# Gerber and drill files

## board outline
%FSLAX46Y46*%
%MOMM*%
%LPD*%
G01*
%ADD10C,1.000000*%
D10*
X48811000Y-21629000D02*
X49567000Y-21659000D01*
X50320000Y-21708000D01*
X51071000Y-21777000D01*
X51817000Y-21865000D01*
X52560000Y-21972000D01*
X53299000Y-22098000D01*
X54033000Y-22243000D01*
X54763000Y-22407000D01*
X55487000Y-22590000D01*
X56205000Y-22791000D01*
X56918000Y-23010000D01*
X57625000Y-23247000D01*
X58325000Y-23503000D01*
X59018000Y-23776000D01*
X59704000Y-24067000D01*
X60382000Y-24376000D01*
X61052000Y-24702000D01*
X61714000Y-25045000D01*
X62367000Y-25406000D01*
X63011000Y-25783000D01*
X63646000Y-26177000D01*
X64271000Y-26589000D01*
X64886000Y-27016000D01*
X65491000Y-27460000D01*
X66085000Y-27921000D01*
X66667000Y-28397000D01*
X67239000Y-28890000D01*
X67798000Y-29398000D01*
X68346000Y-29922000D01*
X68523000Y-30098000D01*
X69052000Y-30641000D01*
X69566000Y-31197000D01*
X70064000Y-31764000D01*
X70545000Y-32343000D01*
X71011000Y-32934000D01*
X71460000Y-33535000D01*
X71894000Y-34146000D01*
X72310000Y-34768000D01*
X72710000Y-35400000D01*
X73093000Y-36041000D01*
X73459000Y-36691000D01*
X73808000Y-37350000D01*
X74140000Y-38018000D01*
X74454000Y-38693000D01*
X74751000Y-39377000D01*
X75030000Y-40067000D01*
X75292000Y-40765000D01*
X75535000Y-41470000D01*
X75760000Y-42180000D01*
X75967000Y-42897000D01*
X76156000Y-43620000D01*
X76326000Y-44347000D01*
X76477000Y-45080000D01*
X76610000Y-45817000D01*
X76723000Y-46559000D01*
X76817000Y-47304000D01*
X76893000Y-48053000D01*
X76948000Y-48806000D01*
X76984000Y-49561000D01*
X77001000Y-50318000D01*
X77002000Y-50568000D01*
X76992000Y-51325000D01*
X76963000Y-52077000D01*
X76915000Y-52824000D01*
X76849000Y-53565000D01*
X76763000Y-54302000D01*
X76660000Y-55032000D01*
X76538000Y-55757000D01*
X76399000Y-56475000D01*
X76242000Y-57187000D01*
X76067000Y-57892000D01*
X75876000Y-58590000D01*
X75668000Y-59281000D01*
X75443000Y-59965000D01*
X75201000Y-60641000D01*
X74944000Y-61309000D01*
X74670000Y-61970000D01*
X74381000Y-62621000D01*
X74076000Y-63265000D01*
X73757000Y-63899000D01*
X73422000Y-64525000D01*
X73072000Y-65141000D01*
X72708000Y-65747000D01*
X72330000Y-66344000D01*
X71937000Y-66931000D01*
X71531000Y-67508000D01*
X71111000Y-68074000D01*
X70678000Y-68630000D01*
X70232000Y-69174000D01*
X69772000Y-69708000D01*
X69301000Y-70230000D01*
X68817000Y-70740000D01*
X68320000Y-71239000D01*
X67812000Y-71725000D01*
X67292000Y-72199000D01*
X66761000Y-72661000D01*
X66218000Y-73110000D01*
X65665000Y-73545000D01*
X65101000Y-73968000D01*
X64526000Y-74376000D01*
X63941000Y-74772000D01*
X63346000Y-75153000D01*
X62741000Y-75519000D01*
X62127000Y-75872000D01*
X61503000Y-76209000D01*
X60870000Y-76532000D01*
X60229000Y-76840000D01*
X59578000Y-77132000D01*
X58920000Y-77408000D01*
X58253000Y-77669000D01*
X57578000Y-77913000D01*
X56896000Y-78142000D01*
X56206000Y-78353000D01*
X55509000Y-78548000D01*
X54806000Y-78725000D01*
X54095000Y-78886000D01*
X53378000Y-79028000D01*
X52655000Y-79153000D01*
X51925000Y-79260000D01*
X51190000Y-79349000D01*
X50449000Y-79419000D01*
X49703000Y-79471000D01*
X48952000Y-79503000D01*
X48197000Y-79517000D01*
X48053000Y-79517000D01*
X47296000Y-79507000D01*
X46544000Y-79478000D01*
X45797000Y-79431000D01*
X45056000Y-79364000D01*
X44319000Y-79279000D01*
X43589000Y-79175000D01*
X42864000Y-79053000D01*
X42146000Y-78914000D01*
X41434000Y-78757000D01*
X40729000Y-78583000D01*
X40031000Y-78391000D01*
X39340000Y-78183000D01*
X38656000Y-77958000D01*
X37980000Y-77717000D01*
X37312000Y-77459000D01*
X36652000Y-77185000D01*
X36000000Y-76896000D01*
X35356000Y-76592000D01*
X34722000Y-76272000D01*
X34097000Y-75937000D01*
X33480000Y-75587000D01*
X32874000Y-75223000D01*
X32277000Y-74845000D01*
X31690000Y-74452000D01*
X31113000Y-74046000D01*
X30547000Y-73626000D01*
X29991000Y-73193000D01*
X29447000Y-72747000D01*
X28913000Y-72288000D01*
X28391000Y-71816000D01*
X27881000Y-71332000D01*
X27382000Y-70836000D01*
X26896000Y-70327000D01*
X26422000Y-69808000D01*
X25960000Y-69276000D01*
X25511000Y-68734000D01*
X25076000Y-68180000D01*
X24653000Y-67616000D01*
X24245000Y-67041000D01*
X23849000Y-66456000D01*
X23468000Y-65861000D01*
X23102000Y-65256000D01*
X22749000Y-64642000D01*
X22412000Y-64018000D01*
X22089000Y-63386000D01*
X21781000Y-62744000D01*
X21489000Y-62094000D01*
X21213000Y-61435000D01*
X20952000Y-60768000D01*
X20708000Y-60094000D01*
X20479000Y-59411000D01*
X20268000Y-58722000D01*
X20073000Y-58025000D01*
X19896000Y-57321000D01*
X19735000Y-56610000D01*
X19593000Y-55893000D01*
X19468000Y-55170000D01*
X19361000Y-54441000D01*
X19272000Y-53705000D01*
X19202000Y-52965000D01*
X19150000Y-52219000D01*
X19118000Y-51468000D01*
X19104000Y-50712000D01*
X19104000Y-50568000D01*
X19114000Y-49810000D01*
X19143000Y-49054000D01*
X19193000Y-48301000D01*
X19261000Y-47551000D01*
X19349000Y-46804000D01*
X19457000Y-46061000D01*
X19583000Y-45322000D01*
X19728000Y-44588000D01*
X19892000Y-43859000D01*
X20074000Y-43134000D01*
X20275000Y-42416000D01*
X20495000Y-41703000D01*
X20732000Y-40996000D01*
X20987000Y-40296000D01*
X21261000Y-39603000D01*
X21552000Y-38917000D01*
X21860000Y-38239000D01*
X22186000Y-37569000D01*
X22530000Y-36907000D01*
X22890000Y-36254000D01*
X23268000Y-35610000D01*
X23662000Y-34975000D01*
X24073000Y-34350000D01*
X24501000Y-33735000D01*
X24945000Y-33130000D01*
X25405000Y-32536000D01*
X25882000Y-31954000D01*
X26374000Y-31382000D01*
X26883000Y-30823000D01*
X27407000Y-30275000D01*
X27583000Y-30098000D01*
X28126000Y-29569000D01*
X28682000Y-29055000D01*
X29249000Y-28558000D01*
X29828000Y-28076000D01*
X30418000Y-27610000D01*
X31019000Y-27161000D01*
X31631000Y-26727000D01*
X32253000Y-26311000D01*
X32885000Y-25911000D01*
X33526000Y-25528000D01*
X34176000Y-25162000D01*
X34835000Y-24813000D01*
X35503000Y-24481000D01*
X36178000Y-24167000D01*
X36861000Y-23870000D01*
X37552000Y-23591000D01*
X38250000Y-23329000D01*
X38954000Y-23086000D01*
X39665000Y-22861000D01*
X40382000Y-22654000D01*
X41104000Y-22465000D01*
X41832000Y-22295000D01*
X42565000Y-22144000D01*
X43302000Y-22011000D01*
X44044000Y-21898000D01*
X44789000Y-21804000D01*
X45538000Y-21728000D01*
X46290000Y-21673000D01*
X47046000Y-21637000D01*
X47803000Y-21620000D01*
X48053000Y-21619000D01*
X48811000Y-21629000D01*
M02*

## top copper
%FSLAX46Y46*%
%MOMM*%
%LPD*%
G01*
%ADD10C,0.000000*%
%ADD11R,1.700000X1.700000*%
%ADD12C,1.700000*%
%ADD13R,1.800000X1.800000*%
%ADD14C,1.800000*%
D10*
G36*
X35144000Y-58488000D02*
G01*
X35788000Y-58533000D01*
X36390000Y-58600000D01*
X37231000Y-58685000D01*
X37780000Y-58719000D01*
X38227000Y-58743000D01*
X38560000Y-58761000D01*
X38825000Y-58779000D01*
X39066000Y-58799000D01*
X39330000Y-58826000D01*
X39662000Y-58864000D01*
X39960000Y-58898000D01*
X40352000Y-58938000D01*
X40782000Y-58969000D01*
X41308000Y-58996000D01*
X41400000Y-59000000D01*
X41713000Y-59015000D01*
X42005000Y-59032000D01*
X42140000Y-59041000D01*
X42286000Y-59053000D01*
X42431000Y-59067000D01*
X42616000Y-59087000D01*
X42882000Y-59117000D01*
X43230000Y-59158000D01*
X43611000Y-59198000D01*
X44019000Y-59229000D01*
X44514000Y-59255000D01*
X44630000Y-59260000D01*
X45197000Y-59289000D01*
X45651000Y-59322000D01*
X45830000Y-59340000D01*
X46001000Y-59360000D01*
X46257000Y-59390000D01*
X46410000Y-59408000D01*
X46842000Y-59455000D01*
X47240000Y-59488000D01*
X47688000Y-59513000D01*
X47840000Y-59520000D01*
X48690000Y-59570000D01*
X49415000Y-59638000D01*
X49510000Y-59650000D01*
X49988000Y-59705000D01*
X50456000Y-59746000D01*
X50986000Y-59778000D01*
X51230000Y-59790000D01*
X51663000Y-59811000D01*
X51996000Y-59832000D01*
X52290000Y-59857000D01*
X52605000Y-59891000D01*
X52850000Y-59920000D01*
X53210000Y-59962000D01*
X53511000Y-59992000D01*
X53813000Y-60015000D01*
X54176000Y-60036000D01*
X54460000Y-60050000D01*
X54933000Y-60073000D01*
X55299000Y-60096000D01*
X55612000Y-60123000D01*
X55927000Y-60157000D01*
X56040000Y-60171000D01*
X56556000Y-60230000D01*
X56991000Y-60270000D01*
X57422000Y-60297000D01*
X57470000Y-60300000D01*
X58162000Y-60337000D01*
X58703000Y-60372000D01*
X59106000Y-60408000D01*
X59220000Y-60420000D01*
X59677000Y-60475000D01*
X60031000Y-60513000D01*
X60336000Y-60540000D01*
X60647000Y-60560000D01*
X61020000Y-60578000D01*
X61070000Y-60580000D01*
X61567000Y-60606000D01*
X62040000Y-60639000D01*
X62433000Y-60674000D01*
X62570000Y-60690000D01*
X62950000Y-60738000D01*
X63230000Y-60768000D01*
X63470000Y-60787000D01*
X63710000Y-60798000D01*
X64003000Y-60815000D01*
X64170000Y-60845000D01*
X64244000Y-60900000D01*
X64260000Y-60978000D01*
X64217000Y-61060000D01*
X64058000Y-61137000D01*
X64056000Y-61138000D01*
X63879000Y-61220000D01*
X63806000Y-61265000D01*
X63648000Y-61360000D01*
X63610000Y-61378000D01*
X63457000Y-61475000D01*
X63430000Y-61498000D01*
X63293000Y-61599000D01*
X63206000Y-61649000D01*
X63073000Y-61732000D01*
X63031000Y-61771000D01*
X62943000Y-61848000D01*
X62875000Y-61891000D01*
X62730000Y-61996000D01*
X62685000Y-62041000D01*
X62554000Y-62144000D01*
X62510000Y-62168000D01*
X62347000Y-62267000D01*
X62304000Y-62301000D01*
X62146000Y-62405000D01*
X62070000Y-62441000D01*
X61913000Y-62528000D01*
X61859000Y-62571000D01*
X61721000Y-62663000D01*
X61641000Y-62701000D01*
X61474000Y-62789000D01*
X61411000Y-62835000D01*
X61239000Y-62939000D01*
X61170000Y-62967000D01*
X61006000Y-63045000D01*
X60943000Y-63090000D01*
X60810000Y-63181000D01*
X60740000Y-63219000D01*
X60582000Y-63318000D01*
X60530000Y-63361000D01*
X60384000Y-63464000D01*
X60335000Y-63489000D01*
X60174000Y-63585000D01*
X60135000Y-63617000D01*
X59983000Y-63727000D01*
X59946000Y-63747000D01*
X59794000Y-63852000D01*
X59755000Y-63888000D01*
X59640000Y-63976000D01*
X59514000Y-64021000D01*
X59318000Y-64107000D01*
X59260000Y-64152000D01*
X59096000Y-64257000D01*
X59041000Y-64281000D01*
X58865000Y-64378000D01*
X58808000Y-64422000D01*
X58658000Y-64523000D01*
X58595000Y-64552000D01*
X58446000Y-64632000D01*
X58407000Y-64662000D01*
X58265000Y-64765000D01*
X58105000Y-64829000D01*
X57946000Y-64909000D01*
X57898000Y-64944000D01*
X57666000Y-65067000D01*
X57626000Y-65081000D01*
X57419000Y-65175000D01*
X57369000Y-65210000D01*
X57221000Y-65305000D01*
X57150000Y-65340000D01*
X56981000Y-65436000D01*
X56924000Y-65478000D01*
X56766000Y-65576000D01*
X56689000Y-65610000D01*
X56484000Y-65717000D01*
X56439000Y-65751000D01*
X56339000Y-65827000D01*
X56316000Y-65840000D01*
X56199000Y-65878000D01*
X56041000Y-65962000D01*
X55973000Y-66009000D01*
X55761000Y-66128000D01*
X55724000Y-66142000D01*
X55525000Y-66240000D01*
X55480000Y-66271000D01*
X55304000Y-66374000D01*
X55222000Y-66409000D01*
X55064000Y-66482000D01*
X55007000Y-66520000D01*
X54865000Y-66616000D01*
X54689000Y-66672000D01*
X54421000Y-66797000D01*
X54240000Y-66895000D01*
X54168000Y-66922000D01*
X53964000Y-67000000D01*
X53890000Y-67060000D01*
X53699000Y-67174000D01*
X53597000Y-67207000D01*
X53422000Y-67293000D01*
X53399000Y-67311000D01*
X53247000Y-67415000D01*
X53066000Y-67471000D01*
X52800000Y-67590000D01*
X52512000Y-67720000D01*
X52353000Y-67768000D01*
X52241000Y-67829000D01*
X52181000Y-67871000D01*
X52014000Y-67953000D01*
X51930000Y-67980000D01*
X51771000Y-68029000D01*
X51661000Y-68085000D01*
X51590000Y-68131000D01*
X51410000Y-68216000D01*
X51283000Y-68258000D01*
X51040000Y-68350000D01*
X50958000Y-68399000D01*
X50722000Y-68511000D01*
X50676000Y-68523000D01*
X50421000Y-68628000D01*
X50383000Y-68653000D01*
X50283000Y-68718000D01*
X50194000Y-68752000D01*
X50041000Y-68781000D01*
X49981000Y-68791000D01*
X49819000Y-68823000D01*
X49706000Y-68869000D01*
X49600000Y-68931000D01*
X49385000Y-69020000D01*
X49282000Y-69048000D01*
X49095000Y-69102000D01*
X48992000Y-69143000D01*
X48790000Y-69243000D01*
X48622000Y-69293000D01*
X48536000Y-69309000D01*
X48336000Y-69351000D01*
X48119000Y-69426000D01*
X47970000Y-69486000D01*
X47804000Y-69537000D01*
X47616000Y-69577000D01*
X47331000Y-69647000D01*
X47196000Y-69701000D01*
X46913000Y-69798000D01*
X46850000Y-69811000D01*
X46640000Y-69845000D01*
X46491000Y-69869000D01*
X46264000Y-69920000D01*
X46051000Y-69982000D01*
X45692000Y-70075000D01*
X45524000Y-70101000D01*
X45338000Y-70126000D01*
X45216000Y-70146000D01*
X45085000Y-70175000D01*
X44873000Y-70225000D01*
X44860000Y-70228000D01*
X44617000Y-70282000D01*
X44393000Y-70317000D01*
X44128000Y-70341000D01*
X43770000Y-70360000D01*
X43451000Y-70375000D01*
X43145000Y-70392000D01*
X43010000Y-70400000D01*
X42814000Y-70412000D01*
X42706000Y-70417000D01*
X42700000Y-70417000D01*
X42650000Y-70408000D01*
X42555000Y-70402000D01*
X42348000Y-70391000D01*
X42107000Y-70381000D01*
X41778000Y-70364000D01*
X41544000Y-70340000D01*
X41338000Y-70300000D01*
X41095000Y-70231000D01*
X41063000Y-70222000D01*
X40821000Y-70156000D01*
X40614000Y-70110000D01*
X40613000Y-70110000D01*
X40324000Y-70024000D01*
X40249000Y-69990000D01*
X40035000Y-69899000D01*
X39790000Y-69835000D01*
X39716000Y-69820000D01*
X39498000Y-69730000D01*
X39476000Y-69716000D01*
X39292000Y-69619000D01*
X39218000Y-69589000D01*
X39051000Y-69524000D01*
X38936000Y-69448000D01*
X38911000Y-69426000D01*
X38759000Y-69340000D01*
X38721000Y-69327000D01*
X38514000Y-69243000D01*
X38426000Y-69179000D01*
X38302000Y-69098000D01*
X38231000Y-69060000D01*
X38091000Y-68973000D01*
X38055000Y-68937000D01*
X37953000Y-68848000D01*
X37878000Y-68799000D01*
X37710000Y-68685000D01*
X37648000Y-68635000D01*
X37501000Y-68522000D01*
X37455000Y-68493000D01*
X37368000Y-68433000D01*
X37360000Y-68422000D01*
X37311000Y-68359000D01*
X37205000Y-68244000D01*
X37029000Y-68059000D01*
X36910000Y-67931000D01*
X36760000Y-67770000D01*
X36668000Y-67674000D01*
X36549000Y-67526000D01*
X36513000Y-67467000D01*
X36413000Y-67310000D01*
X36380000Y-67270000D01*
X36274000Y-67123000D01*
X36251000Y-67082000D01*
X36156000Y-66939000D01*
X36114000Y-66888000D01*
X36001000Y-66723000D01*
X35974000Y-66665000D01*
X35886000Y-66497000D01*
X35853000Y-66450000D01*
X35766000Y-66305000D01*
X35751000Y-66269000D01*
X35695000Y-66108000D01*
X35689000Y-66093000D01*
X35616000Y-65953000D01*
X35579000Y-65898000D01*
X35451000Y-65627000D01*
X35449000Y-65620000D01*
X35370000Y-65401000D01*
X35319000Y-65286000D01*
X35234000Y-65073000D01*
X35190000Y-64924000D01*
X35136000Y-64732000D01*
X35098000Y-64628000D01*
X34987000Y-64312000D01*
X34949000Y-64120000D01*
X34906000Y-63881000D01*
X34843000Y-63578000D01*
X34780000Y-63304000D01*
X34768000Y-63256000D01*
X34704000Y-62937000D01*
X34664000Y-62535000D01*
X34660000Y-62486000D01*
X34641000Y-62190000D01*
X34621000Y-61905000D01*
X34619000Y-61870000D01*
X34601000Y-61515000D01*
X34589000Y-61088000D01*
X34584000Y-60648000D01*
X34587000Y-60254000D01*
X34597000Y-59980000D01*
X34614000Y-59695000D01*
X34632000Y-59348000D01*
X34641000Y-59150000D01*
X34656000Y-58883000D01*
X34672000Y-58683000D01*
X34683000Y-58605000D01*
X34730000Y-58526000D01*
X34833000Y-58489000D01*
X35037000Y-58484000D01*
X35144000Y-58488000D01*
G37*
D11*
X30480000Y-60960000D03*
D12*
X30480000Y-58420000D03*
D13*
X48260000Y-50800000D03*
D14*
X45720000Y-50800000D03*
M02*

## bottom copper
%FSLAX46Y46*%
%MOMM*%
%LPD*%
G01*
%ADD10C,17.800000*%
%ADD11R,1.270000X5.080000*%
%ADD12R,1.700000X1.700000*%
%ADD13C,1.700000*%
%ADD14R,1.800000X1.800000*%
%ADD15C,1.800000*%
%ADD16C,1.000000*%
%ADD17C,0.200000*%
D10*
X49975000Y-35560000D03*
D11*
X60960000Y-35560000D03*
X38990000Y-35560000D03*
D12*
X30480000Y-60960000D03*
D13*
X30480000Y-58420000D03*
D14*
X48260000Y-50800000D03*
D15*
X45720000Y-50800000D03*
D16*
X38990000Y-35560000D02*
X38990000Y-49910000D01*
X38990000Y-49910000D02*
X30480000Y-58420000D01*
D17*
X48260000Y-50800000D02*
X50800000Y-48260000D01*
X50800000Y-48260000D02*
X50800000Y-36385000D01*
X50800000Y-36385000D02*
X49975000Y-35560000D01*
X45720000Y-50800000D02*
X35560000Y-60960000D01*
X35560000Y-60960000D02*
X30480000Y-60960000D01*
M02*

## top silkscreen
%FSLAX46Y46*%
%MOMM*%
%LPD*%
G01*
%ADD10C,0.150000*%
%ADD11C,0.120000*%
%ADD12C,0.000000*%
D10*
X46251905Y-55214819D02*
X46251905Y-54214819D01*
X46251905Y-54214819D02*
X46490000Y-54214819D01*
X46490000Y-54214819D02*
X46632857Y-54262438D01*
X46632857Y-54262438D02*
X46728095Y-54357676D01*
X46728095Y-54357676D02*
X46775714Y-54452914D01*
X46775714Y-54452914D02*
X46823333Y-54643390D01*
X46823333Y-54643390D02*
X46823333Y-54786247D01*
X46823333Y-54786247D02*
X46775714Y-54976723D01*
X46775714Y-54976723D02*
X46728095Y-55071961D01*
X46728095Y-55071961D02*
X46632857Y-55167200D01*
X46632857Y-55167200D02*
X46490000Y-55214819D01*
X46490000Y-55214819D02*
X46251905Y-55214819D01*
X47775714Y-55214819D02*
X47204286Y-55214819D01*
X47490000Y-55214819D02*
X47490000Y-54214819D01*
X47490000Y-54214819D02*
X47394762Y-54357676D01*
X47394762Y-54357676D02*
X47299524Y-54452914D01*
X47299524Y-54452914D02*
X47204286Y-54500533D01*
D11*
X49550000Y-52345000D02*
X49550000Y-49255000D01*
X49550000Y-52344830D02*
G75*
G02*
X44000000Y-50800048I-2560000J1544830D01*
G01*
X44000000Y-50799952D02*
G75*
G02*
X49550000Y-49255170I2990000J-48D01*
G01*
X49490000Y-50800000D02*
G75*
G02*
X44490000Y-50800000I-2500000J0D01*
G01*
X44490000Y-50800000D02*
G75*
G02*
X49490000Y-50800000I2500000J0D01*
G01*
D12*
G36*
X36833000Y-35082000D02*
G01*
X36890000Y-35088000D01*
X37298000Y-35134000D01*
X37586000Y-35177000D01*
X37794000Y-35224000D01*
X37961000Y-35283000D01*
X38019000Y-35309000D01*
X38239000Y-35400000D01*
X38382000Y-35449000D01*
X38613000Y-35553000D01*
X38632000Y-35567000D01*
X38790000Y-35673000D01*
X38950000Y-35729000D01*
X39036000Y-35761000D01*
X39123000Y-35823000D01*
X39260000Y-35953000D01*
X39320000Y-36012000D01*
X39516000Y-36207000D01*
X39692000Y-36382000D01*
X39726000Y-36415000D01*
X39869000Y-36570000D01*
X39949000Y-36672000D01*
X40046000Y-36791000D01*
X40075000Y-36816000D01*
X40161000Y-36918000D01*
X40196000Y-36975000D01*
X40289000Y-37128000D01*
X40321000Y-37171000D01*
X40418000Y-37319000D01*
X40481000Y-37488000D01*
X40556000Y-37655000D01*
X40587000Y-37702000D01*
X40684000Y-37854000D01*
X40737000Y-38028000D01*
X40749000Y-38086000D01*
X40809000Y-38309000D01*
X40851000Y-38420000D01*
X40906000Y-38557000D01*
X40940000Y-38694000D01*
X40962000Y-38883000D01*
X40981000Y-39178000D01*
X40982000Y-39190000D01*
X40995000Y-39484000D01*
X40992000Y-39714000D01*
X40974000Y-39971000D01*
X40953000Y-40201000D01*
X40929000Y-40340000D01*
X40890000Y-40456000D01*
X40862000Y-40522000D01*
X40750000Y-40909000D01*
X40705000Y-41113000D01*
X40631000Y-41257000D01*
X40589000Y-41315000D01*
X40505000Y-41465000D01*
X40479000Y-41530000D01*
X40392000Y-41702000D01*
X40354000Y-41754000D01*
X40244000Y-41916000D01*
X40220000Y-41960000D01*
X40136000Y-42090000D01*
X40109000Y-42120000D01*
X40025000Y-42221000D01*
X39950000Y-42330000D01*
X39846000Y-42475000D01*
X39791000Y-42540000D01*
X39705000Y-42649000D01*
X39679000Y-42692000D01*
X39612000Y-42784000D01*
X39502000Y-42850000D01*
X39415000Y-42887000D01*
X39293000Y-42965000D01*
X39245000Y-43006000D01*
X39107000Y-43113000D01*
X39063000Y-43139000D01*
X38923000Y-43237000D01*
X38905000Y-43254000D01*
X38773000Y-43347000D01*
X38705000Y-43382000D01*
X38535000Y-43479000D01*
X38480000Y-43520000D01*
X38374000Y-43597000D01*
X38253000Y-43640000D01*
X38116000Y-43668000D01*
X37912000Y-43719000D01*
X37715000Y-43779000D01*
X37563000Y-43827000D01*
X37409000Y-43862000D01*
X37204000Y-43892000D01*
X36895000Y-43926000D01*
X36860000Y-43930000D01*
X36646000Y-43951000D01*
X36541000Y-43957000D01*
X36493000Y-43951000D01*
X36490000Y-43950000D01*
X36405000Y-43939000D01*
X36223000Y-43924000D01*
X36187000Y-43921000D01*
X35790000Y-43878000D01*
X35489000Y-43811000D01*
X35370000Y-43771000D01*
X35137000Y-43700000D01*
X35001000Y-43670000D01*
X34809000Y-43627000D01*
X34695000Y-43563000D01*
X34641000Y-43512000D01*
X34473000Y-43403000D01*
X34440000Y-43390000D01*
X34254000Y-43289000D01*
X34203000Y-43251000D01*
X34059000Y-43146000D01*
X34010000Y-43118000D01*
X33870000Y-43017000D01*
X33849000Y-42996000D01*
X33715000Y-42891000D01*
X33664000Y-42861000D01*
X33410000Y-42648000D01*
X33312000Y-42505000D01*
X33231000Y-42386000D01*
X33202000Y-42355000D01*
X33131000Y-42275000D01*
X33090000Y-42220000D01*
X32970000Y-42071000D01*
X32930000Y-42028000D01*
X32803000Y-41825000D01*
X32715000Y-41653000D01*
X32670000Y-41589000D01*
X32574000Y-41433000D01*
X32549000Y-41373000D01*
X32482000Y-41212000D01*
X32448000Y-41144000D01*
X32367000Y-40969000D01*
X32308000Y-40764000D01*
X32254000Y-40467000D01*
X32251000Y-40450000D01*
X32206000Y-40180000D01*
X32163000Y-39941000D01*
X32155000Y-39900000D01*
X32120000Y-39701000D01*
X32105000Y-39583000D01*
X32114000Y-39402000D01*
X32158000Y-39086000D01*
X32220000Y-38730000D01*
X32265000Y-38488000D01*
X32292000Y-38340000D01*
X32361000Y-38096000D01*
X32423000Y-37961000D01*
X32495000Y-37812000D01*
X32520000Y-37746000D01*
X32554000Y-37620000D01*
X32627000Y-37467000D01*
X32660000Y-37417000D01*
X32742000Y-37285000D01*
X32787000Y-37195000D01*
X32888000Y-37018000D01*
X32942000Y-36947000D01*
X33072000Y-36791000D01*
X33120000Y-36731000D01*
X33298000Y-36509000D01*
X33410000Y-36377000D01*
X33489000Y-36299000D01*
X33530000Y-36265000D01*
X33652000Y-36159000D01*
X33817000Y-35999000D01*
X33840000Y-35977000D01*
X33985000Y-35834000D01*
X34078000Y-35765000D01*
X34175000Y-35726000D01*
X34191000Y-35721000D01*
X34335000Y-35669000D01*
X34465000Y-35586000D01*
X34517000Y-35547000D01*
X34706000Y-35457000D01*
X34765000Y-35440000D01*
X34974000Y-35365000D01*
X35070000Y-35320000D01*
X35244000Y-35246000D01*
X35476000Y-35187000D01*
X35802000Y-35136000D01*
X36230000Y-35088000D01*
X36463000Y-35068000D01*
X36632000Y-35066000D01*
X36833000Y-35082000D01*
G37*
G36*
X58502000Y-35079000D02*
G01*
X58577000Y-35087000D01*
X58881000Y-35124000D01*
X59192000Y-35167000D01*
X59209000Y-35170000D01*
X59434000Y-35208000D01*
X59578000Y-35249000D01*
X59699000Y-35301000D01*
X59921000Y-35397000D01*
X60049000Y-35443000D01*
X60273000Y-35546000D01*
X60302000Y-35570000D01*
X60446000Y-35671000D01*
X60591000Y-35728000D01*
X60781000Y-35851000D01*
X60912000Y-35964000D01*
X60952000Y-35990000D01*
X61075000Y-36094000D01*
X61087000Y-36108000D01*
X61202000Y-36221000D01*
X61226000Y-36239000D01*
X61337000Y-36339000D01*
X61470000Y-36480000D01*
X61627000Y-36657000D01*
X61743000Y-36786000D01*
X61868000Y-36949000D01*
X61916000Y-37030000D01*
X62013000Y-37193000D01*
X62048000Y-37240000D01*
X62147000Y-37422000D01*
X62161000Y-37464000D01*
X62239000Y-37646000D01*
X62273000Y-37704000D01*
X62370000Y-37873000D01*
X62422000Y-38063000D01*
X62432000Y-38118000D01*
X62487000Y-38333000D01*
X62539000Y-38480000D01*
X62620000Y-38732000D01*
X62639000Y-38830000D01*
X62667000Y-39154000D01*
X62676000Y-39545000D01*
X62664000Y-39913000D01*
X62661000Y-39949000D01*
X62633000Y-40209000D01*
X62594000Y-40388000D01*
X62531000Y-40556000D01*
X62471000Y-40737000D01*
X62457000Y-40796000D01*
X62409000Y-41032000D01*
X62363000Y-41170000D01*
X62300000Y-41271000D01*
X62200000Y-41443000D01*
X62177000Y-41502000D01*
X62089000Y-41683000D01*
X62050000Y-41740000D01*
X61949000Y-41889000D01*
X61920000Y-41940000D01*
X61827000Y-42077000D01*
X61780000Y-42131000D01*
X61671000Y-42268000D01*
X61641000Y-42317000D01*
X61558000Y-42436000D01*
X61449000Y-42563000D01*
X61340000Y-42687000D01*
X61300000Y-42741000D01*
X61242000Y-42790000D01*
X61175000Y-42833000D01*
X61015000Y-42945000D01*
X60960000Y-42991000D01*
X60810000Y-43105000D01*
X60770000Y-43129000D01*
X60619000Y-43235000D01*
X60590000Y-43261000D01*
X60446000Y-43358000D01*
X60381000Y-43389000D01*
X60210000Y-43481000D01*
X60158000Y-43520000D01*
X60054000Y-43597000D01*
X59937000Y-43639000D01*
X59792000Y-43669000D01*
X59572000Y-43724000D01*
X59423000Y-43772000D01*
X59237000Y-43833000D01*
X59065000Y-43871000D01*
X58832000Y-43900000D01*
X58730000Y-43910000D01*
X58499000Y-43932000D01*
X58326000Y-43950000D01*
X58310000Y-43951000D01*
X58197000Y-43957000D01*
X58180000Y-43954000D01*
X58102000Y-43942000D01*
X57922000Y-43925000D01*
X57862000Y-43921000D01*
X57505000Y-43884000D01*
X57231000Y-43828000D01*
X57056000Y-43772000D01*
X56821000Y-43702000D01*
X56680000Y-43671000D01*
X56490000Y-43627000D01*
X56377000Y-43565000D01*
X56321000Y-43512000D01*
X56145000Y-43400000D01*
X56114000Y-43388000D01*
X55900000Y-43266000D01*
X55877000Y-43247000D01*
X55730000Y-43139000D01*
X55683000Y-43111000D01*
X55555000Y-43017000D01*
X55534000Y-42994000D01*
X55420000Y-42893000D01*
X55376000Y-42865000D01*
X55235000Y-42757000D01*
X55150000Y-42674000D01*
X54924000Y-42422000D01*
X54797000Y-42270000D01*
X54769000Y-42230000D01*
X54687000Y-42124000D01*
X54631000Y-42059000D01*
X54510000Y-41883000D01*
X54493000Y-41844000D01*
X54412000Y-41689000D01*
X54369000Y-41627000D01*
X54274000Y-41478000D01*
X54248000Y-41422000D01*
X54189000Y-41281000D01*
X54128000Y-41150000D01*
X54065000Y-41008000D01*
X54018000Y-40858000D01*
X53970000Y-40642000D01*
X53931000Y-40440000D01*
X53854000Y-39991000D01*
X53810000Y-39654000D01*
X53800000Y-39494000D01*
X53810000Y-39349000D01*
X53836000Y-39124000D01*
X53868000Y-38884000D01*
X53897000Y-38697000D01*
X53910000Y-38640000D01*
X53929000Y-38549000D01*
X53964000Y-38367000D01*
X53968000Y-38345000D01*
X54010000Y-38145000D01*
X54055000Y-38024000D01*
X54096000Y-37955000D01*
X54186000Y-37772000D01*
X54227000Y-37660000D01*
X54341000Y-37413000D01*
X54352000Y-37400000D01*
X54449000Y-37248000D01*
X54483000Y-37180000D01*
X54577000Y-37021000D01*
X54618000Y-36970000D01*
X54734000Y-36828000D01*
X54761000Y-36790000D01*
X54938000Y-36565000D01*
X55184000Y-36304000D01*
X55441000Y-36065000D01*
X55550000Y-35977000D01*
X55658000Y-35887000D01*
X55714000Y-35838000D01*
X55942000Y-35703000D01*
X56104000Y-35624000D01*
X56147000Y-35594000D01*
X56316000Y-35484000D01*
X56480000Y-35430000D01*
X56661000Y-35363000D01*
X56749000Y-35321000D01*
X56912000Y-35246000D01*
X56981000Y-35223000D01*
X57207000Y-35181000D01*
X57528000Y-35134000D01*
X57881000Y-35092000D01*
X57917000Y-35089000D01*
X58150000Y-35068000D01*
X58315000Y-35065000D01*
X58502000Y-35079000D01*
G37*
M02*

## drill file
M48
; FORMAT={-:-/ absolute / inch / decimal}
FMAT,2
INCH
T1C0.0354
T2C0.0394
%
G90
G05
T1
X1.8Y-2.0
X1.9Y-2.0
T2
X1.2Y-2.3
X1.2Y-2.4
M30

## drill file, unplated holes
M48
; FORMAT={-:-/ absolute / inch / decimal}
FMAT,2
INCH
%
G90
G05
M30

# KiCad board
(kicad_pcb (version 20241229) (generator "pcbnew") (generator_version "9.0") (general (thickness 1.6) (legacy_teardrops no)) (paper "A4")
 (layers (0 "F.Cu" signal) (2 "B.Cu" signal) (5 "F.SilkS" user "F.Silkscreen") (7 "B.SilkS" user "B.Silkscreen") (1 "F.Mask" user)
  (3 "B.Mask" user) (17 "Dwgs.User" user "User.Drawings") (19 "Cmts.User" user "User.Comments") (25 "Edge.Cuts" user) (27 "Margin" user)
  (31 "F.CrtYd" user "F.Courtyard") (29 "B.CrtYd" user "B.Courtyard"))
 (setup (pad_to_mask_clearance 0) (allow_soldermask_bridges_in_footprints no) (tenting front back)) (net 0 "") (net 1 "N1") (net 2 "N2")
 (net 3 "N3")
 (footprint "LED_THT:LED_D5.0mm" (layer "F.Cu") (at 48.26 50.8 180)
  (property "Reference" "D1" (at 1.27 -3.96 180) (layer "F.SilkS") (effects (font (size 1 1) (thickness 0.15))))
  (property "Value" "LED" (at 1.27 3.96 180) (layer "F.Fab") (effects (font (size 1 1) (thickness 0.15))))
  (fp_line (start -1.29 -1.545) (end -1.29 1.545) (stroke (width 0.12) (type solid)) (layer "F.SilkS"))
  (fp_arc (start 4.26 0.000048) (mid 2.071756 2.880501) (end -1.29 1.54483) (stroke (width 0.12) (type solid)) (layer "F.SilkS"))
  (fp_arc (start -1.29 -1.54483) (mid 2.071756 -2.880501) (end 4.26 -0.000048) (stroke (width 0.12) (type solid)) (layer "F.SilkS"))
  (fp_circle (center 1.27 0) (end 3.77 0) (stroke (width 0.12) (type solid)) (fill no) (layer "F.SilkS"))
  (pad "1" thru_hole rect (at 0 0 180) (size 1.8 1.8) (drill 0.9) (layers "*.Cu" "*.Mask") (remove_unused_layers no) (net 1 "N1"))
  (pad "2" thru_hole circle (at 2.54 0 180) (size 1.8 1.8) (drill 0.9) (layers "*.Cu" "*.Mask") (remove_unused_layers no) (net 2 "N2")))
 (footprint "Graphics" (layer "F.Cu") (at 0 0)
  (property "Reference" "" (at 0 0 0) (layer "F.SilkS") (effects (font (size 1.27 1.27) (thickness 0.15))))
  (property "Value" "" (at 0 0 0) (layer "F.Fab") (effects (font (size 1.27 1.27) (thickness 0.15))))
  (fp_poly
   (pts (xy 35.144 58.488) (xy 35.788 58.533) (xy 36.39 58.6) (xy 37.231 58.685) (xy 37.78 58.719) (xy 38.227 58.743) (xy 38.56 58.761)
    (xy 38.825 58.779) (xy 39.066 58.799) (xy 39.33 58.826) (xy 39.662 58.864) (xy 39.96 58.898) (xy 40.352 58.938) (xy 40.782 58.969)
    (xy 41.308 58.996) (xy 41.4 59) (xy 41.713 59.015) (xy 42.005 59.032) (xy 42.14 59.041) (xy 42.286 59.053) (xy 42.431 59.067)
    (xy 42.616 59.087) (xy 42.882 59.117) (xy 43.23 59.158) (xy 43.611 59.198) (xy 44.019 59.229) (xy 44.514 59.255) (xy 44.63 59.26)
    (xy 45.197 59.289) (xy 45.651 59.322) (xy 45.83 59.34) (xy 46.001 59.36) (xy 46.257 59.39) (xy 46.41 59.408) (xy 46.842 59.455)
    (xy 47.24 59.488) (xy 47.688 59.513) (xy 47.84 59.52) (xy 48.69 59.57) (xy 49.415 59.638) (xy 49.51 59.65) (xy 49.988 59.705)
    (xy 50.456 59.746) (xy 50.986 59.778) (xy 51.23 59.79) (xy 51.663 59.811) (xy 51.996 59.832) (xy 52.29 59.857) (xy 52.605 59.891)
    (xy 52.85 59.92) (xy 53.21 59.962) (xy 53.511 59.992) (xy 53.813 60.015) (xy 54.176 60.036) (xy 54.46 60.05) (xy 54.933 60.073)
    (xy 55.299 60.096) (xy 55.612 60.123) (xy 55.927 60.157) (xy 56.04 60.171) (xy 56.556 60.23) (xy 56.991 60.27) (xy 57.422 60.297)
    (xy 57.47 60.3) (xy 58.162 60.337) (xy 58.703 60.372) (xy 59.106 60.408) (xy 59.22 60.42) (xy 59.677 60.475) (xy 60.031 60.513)
    (xy 60.336 60.54) (xy 60.647 60.56) (xy 61.02 60.578) (xy 61.07 60.58) (xy 61.567 60.606) (xy 62.04 60.639) (xy 62.433 60.674)
    (xy 62.57 60.69) (xy 62.95 60.738) (xy 63.23 60.768) (xy 63.47 60.787) (xy 63.71 60.798) (xy 64.003 60.815) (xy 64.17 60.845)
    (xy 64.244 60.9) (xy 64.26 60.978) (xy 64.217 61.06) (xy 64.058 61.137) (xy 64.056 61.138) (xy 63.879 61.22) (xy 63.806 61.265)
    (xy 63.648 61.36) (xy 63.61 61.378) (xy 63.457 61.475) (xy 63.43 61.498) (xy 63.293 61.599) (xy 63.206 61.649) (xy 63.073 61.732)
    (xy 63.031 61.771) (xy 62.943 61.848) (xy 62.875 61.891) (xy 62.73 61.996) (xy 62.685 62.041) (xy 62.554 62.144) (xy 62.51 62.168)
    (xy 62.347 62.267) (xy 62.304 62.301) (xy 62.146 62.405) (xy 62.07 62.441) (xy 61.913 62.528) (xy 61.859 62.571) (xy 61.721 62.663)
    (xy 61.641 62.701) (xy 61.474 62.789) (xy 61.411 62.835) (xy 61.239 62.939) (xy 61.17 62.967) (xy 61.006 63.045) (xy 60.943 63.09)
    (xy 60.81 63.181) (xy 60.74 63.219) (xy 60.582 63.318) (xy 60.53 63.361) (xy 60.384 63.464) (xy 60.335 63.489) (xy 60.174 63.585)
    (xy 60.135 63.617) (xy 59.983 63.727) (xy 59.946 63.747) (xy 59.794 63.852) (xy 59.755 63.888) (xy 59.64 63.976) (xy 59.514 64.021)
    (xy 59.318 64.107) (xy 59.26 64.152) (xy 59.096 64.257) (xy 59.041 64.281) (xy 58.865 64.378) (xy 58.808 64.422) (xy 58.658 64.523)
    (xy 58.595 64.552) (xy 58.446 64.632) (xy 58.407 64.662) (xy 58.265 64.765) (xy 58.105 64.829) (xy 57.946 64.909) (xy 57.898 64.944)
    (xy 57.666 65.067) (xy 57.626 65.081) (xy 57.419 65.175) (xy 57.369 65.21) (xy 57.221 65.305) (xy 57.15 65.34) (xy 56.981 65.436)
    (xy 56.924 65.478) (xy 56.766 65.576) (xy 56.689 65.61) (xy 56.484 65.717) (xy 56.439 65.751) (xy 56.339 65.827) (xy 56.316 65.84)
    (xy 56.199 65.878) (xy 56.041 65.962) (xy 55.973 66.009) (xy 55.761 66.128) (xy 55.724 66.142) (xy 55.525 66.24) (xy 55.48 66.271)
    (xy 55.304 66.374) (xy 55.222 66.409) (xy 55.064 66.482) (xy 55.007 66.52) (xy 54.865 66.616) (xy 54.689 66.672) (xy 54.421 66.797)
    (xy 54.24 66.895) (xy 54.168 66.922) (xy 53.964 67) (xy 53.89 67.06) (xy 53.699 67.174) (xy 53.597 67.207) (xy 53.422 67.293)
    (xy 53.399 67.311) (xy 53.247 67.415) (xy 53.066 67.471) (xy 52.8 67.59) (xy 52.512 67.72) (xy 52.353 67.768) (xy 52.241 67.829)
    (xy 52.181 67.871) (xy 52.014 67.953) (xy 51.93 67.98) (xy 51.771 68.029) (xy 51.661 68.085) (xy 51.59 68.131) (xy 51.41 68.216)
    (xy 51.283 68.258) (xy 51.04 68.35) (xy 50.958 68.399) (xy 50.722 68.511) (xy 50.676 68.523) (xy 50.421 68.628) (xy 50.383 68.653)
    (xy 50.283 68.718) (xy 50.194 68.752) (xy 50.041 68.781) (xy 49.981 68.791) (xy 49.819 68.823) (xy 49.706 68.869) (xy 49.6 68.931)
    (xy 49.385 69.02) (xy 49.282 69.048) (xy 49.095 69.102) (xy 48.992 69.143) (xy 48.79 69.243) (xy 48.622 69.293) (xy 48.536 69.309)
    (xy 48.336 69.351) (xy 48.119 69.426) (xy 47.97 69.486) (xy 47.804 69.537) (xy 47.616 69.577) (xy 47.331 69.647) (xy 47.196 69.701)
    (xy 46.913 69.798) (xy 46.85 69.811) (xy 46.64 69.845) (xy 46.491 69.869) (xy 46.264 69.92) (xy 46.051 69.982) (xy 45.692 70.075)
    (xy 45.524 70.101) (xy 45.338 70.126) (xy 45.216 70.146) (xy 45.085 70.175) (xy 44.873 70.225) (xy 44.86 70.228) (xy 44.617 70.282)
    (xy 44.393 70.317) (xy 44.128 70.341) (xy 43.77 70.36) (xy 43.451 70.375) (xy 43.145 70.392) (xy 43.01 70.4) (xy 42.814 70.412)
    (xy 42.706 70.417) (xy 42.7 70.417) (xy 42.65 70.408) (xy 42.555 70.402) (xy 42.348 70.391) (xy 42.107 70.381) (xy 41.778 70.364)
    (xy 41.544 70.34) (xy 41.338 70.3) (xy 41.095 70.231) (xy 41.063 70.222) (xy 40.821 70.156) (xy 40.614 70.11) (xy 40.613 70.11)
    (xy 40.324 70.024) (xy 40.249 69.99) (xy 40.035 69.899) (xy 39.79 69.835) (xy 39.716 69.82) (xy 39.498 69.73) (xy 39.476 69.716)
    (xy 39.292 69.619) (xy 39.218 69.589) (xy 39.051 69.524) (xy 38.936 69.448) (xy 38.911 69.426) (xy 38.759 69.34) (xy 38.721 69.327)
    (xy 38.514 69.243) (xy 38.426 69.179) (xy 38.302 69.098) (xy 38.231 69.06) (xy 38.091 68.973) (xy 38.055 68.937) (xy 37.953 68.848)
    (xy 37.878 68.799) (xy 37.71 68.685) (xy 37.648 68.635) (xy 37.501 68.522) (xy 37.455 68.493) (xy 37.368 68.433) (xy 37.36 68.422)
    (xy 37.311 68.359) (xy 37.205 68.244) (xy 37.029 68.059) (xy 36.91 67.931) (xy 36.76 67.77) (xy 36.668 67.674) (xy 36.549 67.526)
    (xy 36.513 67.467) (xy 36.413 67.31) (xy 36.38 67.27) (xy 36.274 67.123) (xy 36.251 67.082) (xy 36.156 66.939) (xy 36.114 66.888)
    (xy 36.001 66.723) (xy 35.974 66.665) (xy 35.886 66.497) (xy 35.853 66.45) (xy 35.766 66.305) (xy 35.751 66.269) (xy 35.695 66.108)
    (xy 35.689 66.093) (xy 35.616 65.953) (xy 35.579 65.898) (xy 35.451 65.627) (xy 35.449 65.62) (xy 35.37 65.401) (xy 35.319 65.286)
    (xy 35.234 65.073) (xy 35.19 64.924) (xy 35.136 64.732) (xy 35.098 64.628) (xy 34.987 64.312) (xy 34.949 64.12) (xy 34.906 63.881)
    (xy 34.843 63.578) (xy 34.78 63.304) (xy 34.768 63.256) (xy 34.704 62.937) (xy 34.664 62.535) (xy 34.66 62.486) (xy 34.641 62.19)
    (xy 34.621 61.905) (xy 34.619 61.87) (xy 34.601 61.515) (xy 34.589 61.088) (xy 34.584 60.648) (xy 34.587 60.254) (xy 34.597 59.98)
    (xy 34.614 59.695) (xy 34.632 59.348) (xy 34.641 59.15) (xy 34.656 58.883) (xy 34.672 58.683) (xy 34.683 58.605) (xy 34.73 58.526)
    (xy 34.833 58.489) (xy 35.037 58.484))
   (stroke (width 0) (type solid)) (fill yes) (layer "F.Cu")))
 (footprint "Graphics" (layer "F.Cu") (at 0 0)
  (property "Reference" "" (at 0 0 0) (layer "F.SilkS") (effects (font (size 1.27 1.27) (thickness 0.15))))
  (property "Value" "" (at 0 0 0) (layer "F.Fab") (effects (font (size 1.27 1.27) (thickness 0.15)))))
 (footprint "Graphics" (layer "F.Cu") (at 0 0)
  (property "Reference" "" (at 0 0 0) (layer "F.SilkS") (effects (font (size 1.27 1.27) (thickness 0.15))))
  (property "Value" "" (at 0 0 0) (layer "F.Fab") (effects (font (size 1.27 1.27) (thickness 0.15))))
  (fp_poly
   (pts (xy 58.502 35.079) (xy 58.577 35.087) (xy 58.881 35.124) (xy 59.192 35.167) (xy 59.209 35.17) (xy 59.434 35.208) (xy 59.578 35.249)
    (xy 59.699 35.301) (xy 59.921 35.397) (xy 60.049 35.443) (xy 60.273 35.546) (xy 60.302 35.57) (xy 60.446 35.671) (xy 60.591 35.728)
    (xy 60.781 35.851) (xy 60.912 35.964) (xy 60.952 35.99) (xy 61.075 36.094) (xy 61.087 36.108) (xy 61.202 36.221) (xy 61.226 36.239)
    (xy 61.337 36.339) (xy 61.47 36.48) (xy 61.627 36.657) (xy 61.743 36.786) (xy 61.868 36.949) (xy 61.916 37.03) (xy 62.013 37.193)
    (xy 62.048 37.24) (xy 62.147 37.422) (xy 62.161 37.464) (xy 62.239 37.646) (xy 62.273 37.704) (xy 62.37 37.873) (xy 62.422 38.063)
    (xy 62.432 38.118) (xy 62.487 38.333) (xy 62.539 38.48) (xy 62.62 38.732) (xy 62.639 38.83) (xy 62.667 39.154) (xy 62.676 39.545)
    (xy 62.664 39.913) (xy 62.661 39.949) (xy 62.633 40.209) (xy 62.594 40.388) (xy 62.531 40.556) (xy 62.471 40.737) (xy 62.457 40.796)
    (xy 62.409 41.032) (xy 62.363 41.17) (xy 62.3 41.271) (xy 62.2 41.443) (xy 62.177 41.502) (xy 62.089 41.683) (xy 62.05 41.74)
    (xy 61.949 41.889) (xy 61.92 41.94) (xy 61.827 42.077) (xy 61.78 42.131) (xy 61.671 42.268) (xy 61.641 42.317) (xy 61.558 42.436)
    (xy 61.449 42.563) (xy 61.34 42.687) (xy 61.3 42.741) (xy 61.242 42.79) (xy 61.175 42.833) (xy 61.015 42.945) (xy 60.96 42.991)
    (xy 60.81 43.105) (xy 60.77 43.129) (xy 60.619 43.235) (xy 60.59 43.261) (xy 60.446 43.358) (xy 60.381 43.389) (xy 60.21 43.481)
    (xy 60.158 43.52) (xy 60.054 43.597) (xy 59.937 43.639) (xy 59.792 43.669) (xy 59.572 43.724) (xy 59.423 43.772) (xy 59.237 43.833)
    (xy 59.065 43.871) (xy 58.832 43.9) (xy 58.73 43.91) (xy 58.499 43.932) (xy 58.326 43.95) (xy 58.31 43.951) (xy 58.197 43.957)
    (xy 58.18 43.954) (xy 58.102 43.942) (xy 57.922 43.925) (xy 57.862 43.921) (xy 57.505 43.884) (xy 57.231 43.828) (xy 57.056 43.772)
    (xy 56.821 43.702) (xy 56.68 43.671) (xy 56.49 43.627) (xy 56.377 43.565) (xy 56.321 43.512) (xy 56.145 43.4) (xy 56.114 43.388)
    (xy 55.9 43.266) (xy 55.877 43.247) (xy 55.73 43.139) (xy 55.683 43.111) (xy 55.555 43.017) (xy 55.534 42.994) (xy 55.42 42.893)
    (xy 55.376 42.865) (xy 55.235 42.757) (xy 55.15 42.674) (xy 54.924 42.422) (xy 54.797 42.27) (xy 54.769 42.23) (xy 54.687 42.124)
    (xy 54.631 42.059) (xy 54.51 41.883) (xy 54.493 41.844) (xy 54.412 41.689) (xy 54.369 41.627) (xy 54.274 41.478) (xy 54.248 41.422)
    (xy 54.189 41.281) (xy 54.128 41.15) (xy 54.065 41.008) (xy 54.018 40.858) (xy 53.97 40.642) (xy 53.931 40.44) (xy 53.854 39.991)
    (xy 53.81 39.654) (xy 53.8 39.494) (xy 53.81 39.349) (xy 53.836 39.124) (xy 53.868 38.884) (xy 53.897 38.697) (xy 53.91 38.64)
    (xy 53.929 38.549) (xy 53.964 38.367) (xy 53.968 38.345) (xy 54.01 38.145) (xy 54.055 38.024) (xy 54.096 37.955) (xy 54.186 37.772)
    (xy 54.227 37.66) (xy 54.341 37.413) (xy 54.352 37.4) (xy 54.449 37.248) (xy 54.483 37.18) (xy 54.577 37.021) (xy 54.618 36.97)
    (xy 54.734 36.828) (xy 54.761 36.79) (xy 54.938 36.565) (xy 55.184 36.304) (xy 55.441 36.065) (xy 55.55 35.977) (xy 55.658 35.887)
    (xy 55.714 35.838) (xy 55.942 35.703) (xy 56.104 35.624) (xy 56.147 35.594) (xy 56.316 35.484) (xy 56.48 35.43) (xy 56.661 35.363)
    (xy 56.749 35.321) (xy 56.912 35.246) (xy 56.981 35.223) (xy 57.207 35.181) (xy 57.528 35.134) (xy 57.881 35.092) (xy 57.917 35.089)
    (xy 58.15 35.068) (xy 58.315 35.065))
   (stroke (width 0) (type solid)) (fill yes) (layer "F.SilkS"))
  (fp_poly
   (pts (xy 36.833 35.082) (xy 36.89 35.088) (xy 37.298 35.134) (xy 37.586 35.177) (xy 37.794 35.224) (xy 37.961 35.283) (xy 38.019 35.309)
    (xy 38.239 35.4) (xy 38.382 35.449) (xy 38.613 35.553) (xy 38.632 35.567) (xy 38.79 35.673) (xy 38.95 35.729) (xy 39.036 35.761)
    (xy 39.123 35.823) (xy 39.26 35.953) (xy 39.32 36.012) (xy 39.516 36.207) (xy 39.692 36.382) (xy 39.726 36.415) (xy 39.869 36.57)
    (xy 39.949 36.672) (xy 40.046 36.791) (xy 40.075 36.816) (xy 40.161 36.918) (xy 40.196 36.975) (xy 40.289 37.128) (xy 40.321 37.171)
    (xy 40.418 37.319) (xy 40.481 37.488) (xy 40.556 37.655) (xy 40.587 37.702) (xy 40.684 37.854) (xy 40.737 38.028) (xy 40.749 38.086)
    (xy 40.809 38.309) (xy 40.851 38.42) (xy 40.906 38.557) (xy 40.94 38.694) (xy 40.962 38.883) (xy 40.981 39.178) (xy 40.982 39.19)
    (xy 40.995 39.484) (xy 40.992 39.714) (xy 40.974 39.971) (xy 40.953 40.201) (xy 40.929 40.34) (xy 40.89 40.456) (xy 40.862 40.522)
    (xy 40.75 40.909) (xy 40.705 41.113) (xy 40.631 41.257) (xy 40.589 41.315) (xy 40.505 41.465) (xy 40.479 41.53) (xy 40.392 41.702)
    (xy 40.354 41.754) (xy 40.244 41.916) (xy 40.22 41.96) (xy 40.136 42.09) (xy 40.109 42.12) (xy 40.025 42.221) (xy 39.95 42.33)
    (xy 39.846 42.475) (xy 39.791 42.54) (xy 39.705 42.649) (xy 39.679 42.692) (xy 39.612 42.784) (xy 39.502 42.85) (xy 39.415 42.887)
    (xy 39.293 42.965) (xy 39.245 43.006) (xy 39.107 43.113) (xy 39.063 43.139) (xy 38.923 43.237) (xy 38.905 43.254) (xy 38.773 43.347)
    (xy 38.705 43.382) (xy 38.535 43.479) (xy 38.48 43.52) (xy 38.374 43.597) (xy 38.253 43.64) (xy 38.116 43.668) (xy 37.912 43.719)
    (xy 37.715 43.779) (xy 37.563 43.827) (xy 37.409 43.862) (xy 37.204 43.892) (xy 36.895 43.926) (xy 36.86 43.93) (xy 36.646 43.951)
    (xy 36.541 43.957) (xy 36.493 43.951) (xy 36.49 43.95) (xy 36.405 43.939) (xy 36.223 43.924) (xy 36.187 43.921) (xy 35.79 43.878)
    (xy 35.489 43.811) (xy 35.37 43.771) (xy 35.137 43.7) (xy 35.001 43.67) (xy 34.809 43.627) (xy 34.695 43.563) (xy 34.641 43.512)
    (xy 34.473 43.403) (xy 34.44 43.39) (xy 34.254 43.289) (xy 34.203 43.251) (xy 34.059 43.146) (xy 34.01 43.118) (xy 33.87 43.017)
    (xy 33.849 42.996) (xy 33.715 42.891) (xy 33.664 42.861) (xy 33.41 42.648) (xy 33.312 42.505) (xy 33.231 42.386) (xy 33.202 42.355)
    (xy 33.131 42.275) (xy 33.09 42.22) (xy 32.97 42.071) (xy 32.93 42.028) (xy 32.803 41.825) (xy 32.715 41.653) (xy 32.67 41.589)
    (xy 32.574 41.433) (xy 32.549 41.373) (xy 32.482 41.212) (xy 32.448 41.144) (xy 32.367 40.969) (xy 32.308 40.764) (xy 32.254 40.467)
    (xy 32.251 40.45) (xy 32.206 40.18) (xy 32.163 39.941) (xy 32.155 39.9) (xy 32.12 39.701) (xy 32.105 39.583) (xy 32.114 39.402)
    (xy 32.158 39.086) (xy 32.22 38.73) (xy 32.265 38.488) (xy 32.292 38.34) (xy 32.361 38.096) (xy 32.423 37.961) (xy 32.495 37.812)
    (xy 32.52 37.746) (xy 32.554 37.62) (xy 32.627 37.467) (xy 32.66 37.417) (xy 32.742 37.285) (xy 32.787 37.195) (xy 32.888 37.018)
    (xy 32.942 36.947) (xy 33.072 36.791) (xy 33.12 36.731) (xy 33.298 36.509) (xy 33.41 36.377) (xy 33.489 36.299) (xy 33.53 36.265)
    (xy 33.652 36.159) (xy 33.817 35.999) (xy 33.84 35.977) (xy 33.985 35.834) (xy 34.078 35.765) (xy 34.175 35.726) (xy 34.191 35.721)
    (xy 34.335 35.669) (xy 34.465 35.586) (xy 34.517 35.547) (xy 34.706 35.457) (xy 34.765 35.44) (xy 34.974 35.365) (xy 35.07 35.32)
    (xy 35.244 35.246) (xy 35.476 35.187) (xy 35.802 35.136) (xy 36.23 35.088) (xy 36.463 35.068) (xy 36.632 35.066))
   (stroke (width 0) (type solid)) (fill yes) (layer "F.SilkS")))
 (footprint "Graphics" (layer "F.Cu") (at 0 0)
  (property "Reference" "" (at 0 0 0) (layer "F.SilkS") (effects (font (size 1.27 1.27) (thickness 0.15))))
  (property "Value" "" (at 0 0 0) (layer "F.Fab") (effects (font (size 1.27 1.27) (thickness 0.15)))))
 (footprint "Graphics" (layer "F.Cu") (at 0 0)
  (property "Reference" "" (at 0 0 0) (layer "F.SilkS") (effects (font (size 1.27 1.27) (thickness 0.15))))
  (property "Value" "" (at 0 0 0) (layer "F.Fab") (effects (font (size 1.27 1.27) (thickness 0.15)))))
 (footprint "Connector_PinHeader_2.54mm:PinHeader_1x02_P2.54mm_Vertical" (layer "B.Cu") (at 30.48 60.96)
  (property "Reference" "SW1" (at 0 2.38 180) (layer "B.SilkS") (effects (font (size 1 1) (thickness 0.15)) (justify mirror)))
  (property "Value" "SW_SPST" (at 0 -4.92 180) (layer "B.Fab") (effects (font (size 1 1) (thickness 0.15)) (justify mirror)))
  (pad "1" thru_hole rect (at 0 0) (size 1.7 1.7) (drill 1) (layers "*.Cu" "*.Mask") (remove_unused_layers no) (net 2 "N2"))
  (pad "2" thru_hole circle (at 0 -2.54) (size 1.7 1.7) (drill 1) (layers "*.Cu" "*.Mask") (remove_unused_layers no) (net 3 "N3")))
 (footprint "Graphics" (layer "B.Cu") (at 0 0)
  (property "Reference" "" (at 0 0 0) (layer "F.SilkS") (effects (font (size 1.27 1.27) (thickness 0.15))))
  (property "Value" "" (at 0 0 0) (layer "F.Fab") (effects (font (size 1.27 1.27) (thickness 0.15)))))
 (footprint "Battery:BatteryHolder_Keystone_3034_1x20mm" (layer "B.Cu") (at 49.975 35.56)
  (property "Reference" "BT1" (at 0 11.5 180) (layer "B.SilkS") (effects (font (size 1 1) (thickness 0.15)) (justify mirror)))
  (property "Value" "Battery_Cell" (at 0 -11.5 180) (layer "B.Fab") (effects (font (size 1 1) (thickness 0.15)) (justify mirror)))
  (pad "1" smd rect (at -10.985 0) (size 1.27 5.08) (layers "B.Cu" "B.Mask" "B.Paste") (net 3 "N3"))
  (pad "1" smd rect (at 10.985 0) (size 1.27 5.08) (layers "B.Cu" "B.Mask" "B.Paste") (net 3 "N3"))
  (pad "2" smd circle (at 0 0) (size 17.8 17.8) (layers "B.Cu" "B.Mask") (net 1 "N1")))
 (gr_poly
  (pts (xy 77.002 50.568) (xy 76.992 51.325) (xy 76.963 52.077) (xy 76.915 52.824) (xy 76.849 53.565) (xy 76.763 54.302) (xy 76.66 55.032)
   (xy 76.538 55.757) (xy 76.399 56.475) (xy 76.242 57.187) (xy 76.067 57.892) (xy 75.876 58.59) (xy 75.668 59.281) (xy 75.443 59.965)
   (xy 75.201 60.641) (xy 74.944 61.309) (xy 74.67 61.97) (xy 74.381 62.621) (xy 74.076 63.265) (xy 73.757 63.899) (xy 73.422 64.525)
   (xy 73.072 65.141) (xy 72.708 65.747) (xy 72.33 66.344) (xy 71.937 66.931) (xy 71.531 67.508) (xy 71.111 68.074) (xy 70.678 68.63)
   (xy 70.232 69.174) (xy 69.772 69.708) (xy 69.301 70.23) (xy 68.817 70.74) (xy 68.32 71.239) (xy 67.812 71.725) (xy 67.292 72.199)
   (xy 66.761 72.661) (xy 66.218 73.11) (xy 65.665 73.545) (xy 65.101 73.968) (xy 64.526 74.376) (xy 63.941 74.772) (xy 63.346 75.153)
   (xy 62.741 75.519) (xy 62.127 75.872) (xy 61.503 76.209) (xy 60.87 76.532) (xy 60.229 76.84) (xy 59.578 77.132) (xy 58.92 77.408)
   (xy 58.253 77.669) (xy 57.578 77.913) (xy 56.896 78.142) (xy 56.206 78.353) (xy 55.509 78.548) (xy 54.806 78.725) (xy 54.095 78.886)
   (xy 53.378 79.028) (xy 52.655 79.153) (xy 51.925 79.26) (xy 51.19 79.349) (xy 50.449 79.419) (xy 49.703 79.471) (xy 48.952 79.503)
   (xy 48.197 79.517) (xy 48.053 79.517) (xy 47.296 79.507) (xy 46.544 79.478) (xy 45.797 79.431) (xy 45.056 79.364) (xy 44.319 79.279)
   (xy 43.589 79.175) (xy 42.864 79.053) (xy 42.146 78.914) (xy 41.434 78.757) (xy 40.729 78.583) (xy 40.031 78.391) (xy 39.34 78.183)
   (xy 38.656 77.958) (xy 37.98 77.717) (xy 37.312 77.459) (xy 36.652 77.185) (xy 36 76.896) (xy 35.356 76.592) (xy 34.722 76.272)
   (xy 34.097 75.937) (xy 33.48 75.587) (xy 32.874 75.223) (xy 32.277 74.845) (xy 31.69 74.452) (xy 31.113 74.046) (xy 30.547 73.626)
   (xy 29.991 73.193) (xy 29.447 72.747) (xy 28.913 72.288) (xy 28.391 71.816) (xy 27.881 71.332) (xy 27.382 70.836) (xy 26.896 70.327)
   (xy 26.422 69.808) (xy 25.96 69.276) (xy 25.511 68.734) (xy 25.076 68.18) (xy 24.653 67.616) (xy 24.245 67.041) (xy 23.849 66.456)
   (xy 23.468 65.861) (xy 23.102 65.256) (xy 22.749 64.642) (xy 22.412 64.018) (xy 22.089 63.386) (xy 21.781 62.744) (xy 21.489 62.094)
   (xy 21.213 61.435) (xy 20.952 60.768) (xy 20.708 60.094) (xy 20.479 59.411) (xy 20.268 58.722) (xy 20.073 58.025) (xy 19.896 57.321)
   (xy 19.735 56.61) (xy 19.593 55.893) (xy 19.468 55.17) (xy 19.361 54.441) (xy 19.272 53.705) (xy 19.202 52.965) (xy 19.15 52.219)
   (xy 19.118 51.468) (xy 19.104 50.712) (xy 19.104 50.568) (xy 19.114 49.81) (xy 19.143 49.054) (xy 19.193 48.301) (xy 19.261 47.551)
   (xy 19.349 46.804) (xy 19.457 46.061) (xy 19.583 45.322) (xy 19.728 44.588) (xy 19.892 43.859) (xy 20.074 43.134) (xy 20.275 42.416)
   (xy 20.495 41.703) (xy 20.732 40.996) (xy 20.987 40.296) (xy 21.261 39.603) (xy 21.552 38.917) (xy 21.86 38.239) (xy 22.186 37.569)
   (xy 22.53 36.907) (xy 22.89 36.254) (xy 23.268 35.61) (xy 23.662 34.975) (xy 24.073 34.35) (xy 24.501 33.735) (xy 24.945 33.13)
   (xy 25.405 32.536) (xy 25.882 31.954) (xy 26.374 31.382) (xy 26.883 30.823) (xy 27.407 30.275) (xy 27.583 30.098) (xy 28.126 29.569)
   (xy 28.682 29.055) (xy 29.249 28.558) (xy 29.828 28.076) (xy 30.418 27.61) (xy 31.019 27.161) (xy 31.631 26.727) (xy 32.253 26.311)
   (xy 32.885 25.911) (xy 33.526 25.528) (xy 34.176 25.162) (xy 34.835 24.813) (xy 35.503 24.481) (xy 36.178 24.167) (xy 36.861 23.87)
   (xy 37.552 23.591) (xy 38.25 23.329) (xy 38.954 23.086) (xy 39.665 22.861) (xy 40.382 22.654) (xy 41.104 22.465) (xy 41.832 22.295)
   (xy 42.565 22.144) (xy 43.302 22.011) (xy 44.044 21.898) (xy 44.789 21.804) (xy 45.538 21.728) (xy 46.29 21.673) (xy 47.046 21.637)
   (xy 47.803 21.62) (xy 48.053 21.619) (xy 48.811 21.629) (xy 49.567 21.659) (xy 50.32 21.708) (xy 51.071 21.777) (xy 51.817 21.865)
   (xy 52.56 21.972) (xy 53.299 22.098) (xy 54.033 22.243) (xy 54.763 22.407) (xy 55.487 22.59) (xy 56.205 22.791) (xy 56.918 23.01)
   (xy 57.625 23.247) (xy 58.325 23.503) (xy 59.018 23.776) (xy 59.704 24.067) (xy 60.382 24.376) (xy 61.052 24.702) (xy 61.714 25.045)
   (xy 62.367 25.406) (xy 63.011 25.783) (xy 63.646 26.177) (xy 64.271 26.589) (xy 64.886 27.016) (xy 65.491 27.46) (xy 66.085 27.921)
   (xy 66.667 28.397) (xy 67.239 28.89) (xy 67.798 29.398) (xy 68.346 29.922) (xy 68.523 30.098) (xy 69.052 30.641) (xy 69.566 31.197)
   (xy 70.064 31.764) (xy 70.545 32.343) (xy 71.011 32.934) (xy 71.46 33.535) (xy 71.894 34.146) (xy 72.31 34.768) (xy 72.71 35.4)
   (xy 73.093 36.041) (xy 73.459 36.691) (xy 73.808 37.35) (xy 74.14 38.018) (xy 74.454 38.693) (xy 74.751 39.377) (xy 75.03 40.067)
   (xy 75.292 40.765) (xy 75.535 41.47) (xy 75.76 42.18) (xy 75.967 42.897) (xy 76.156 43.62) (xy 76.326 44.347) (xy 76.477 45.08)
   (xy 76.61 45.817) (xy 76.723 46.559) (xy 76.817 47.304) (xy 76.893 48.053) (xy 76.948 48.806) (xy 76.984 49.561) (xy 77.001 50.318)
   (xy 77.002 50.568))
  (stroke (width 1) (type solid)) (fill no) (layer "Edge.Cuts"))
 (segment (start 38.99 49.91) (end 30.48 58.42) (width 1) (layer "B.Cu") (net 3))
 (segment (start 38.99 35.56) (end 38.99 49.91) (width 1) (layer "B.Cu") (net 3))
 (segment (start 50.8 36.385) (end 49.975 35.56) (width 0.2) (layer "B.Cu") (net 1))
 (segment (start 50.8 48.26) (end 50.8 36.385) (width 0.2) (layer "B.Cu") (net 1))
 (segment (start 48.26 50.8) (end 50.8 48.26) (width 0.2) (layer "B.Cu") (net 1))
 (segment (start 45.72 50.8) (end 35.56 60.96) (width 0.2) (layer "B.Cu") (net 2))
 (segment (start 35.56 60.96) (end 30.48 60.96) (width 0.2) (layer "B.Cu") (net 2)))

